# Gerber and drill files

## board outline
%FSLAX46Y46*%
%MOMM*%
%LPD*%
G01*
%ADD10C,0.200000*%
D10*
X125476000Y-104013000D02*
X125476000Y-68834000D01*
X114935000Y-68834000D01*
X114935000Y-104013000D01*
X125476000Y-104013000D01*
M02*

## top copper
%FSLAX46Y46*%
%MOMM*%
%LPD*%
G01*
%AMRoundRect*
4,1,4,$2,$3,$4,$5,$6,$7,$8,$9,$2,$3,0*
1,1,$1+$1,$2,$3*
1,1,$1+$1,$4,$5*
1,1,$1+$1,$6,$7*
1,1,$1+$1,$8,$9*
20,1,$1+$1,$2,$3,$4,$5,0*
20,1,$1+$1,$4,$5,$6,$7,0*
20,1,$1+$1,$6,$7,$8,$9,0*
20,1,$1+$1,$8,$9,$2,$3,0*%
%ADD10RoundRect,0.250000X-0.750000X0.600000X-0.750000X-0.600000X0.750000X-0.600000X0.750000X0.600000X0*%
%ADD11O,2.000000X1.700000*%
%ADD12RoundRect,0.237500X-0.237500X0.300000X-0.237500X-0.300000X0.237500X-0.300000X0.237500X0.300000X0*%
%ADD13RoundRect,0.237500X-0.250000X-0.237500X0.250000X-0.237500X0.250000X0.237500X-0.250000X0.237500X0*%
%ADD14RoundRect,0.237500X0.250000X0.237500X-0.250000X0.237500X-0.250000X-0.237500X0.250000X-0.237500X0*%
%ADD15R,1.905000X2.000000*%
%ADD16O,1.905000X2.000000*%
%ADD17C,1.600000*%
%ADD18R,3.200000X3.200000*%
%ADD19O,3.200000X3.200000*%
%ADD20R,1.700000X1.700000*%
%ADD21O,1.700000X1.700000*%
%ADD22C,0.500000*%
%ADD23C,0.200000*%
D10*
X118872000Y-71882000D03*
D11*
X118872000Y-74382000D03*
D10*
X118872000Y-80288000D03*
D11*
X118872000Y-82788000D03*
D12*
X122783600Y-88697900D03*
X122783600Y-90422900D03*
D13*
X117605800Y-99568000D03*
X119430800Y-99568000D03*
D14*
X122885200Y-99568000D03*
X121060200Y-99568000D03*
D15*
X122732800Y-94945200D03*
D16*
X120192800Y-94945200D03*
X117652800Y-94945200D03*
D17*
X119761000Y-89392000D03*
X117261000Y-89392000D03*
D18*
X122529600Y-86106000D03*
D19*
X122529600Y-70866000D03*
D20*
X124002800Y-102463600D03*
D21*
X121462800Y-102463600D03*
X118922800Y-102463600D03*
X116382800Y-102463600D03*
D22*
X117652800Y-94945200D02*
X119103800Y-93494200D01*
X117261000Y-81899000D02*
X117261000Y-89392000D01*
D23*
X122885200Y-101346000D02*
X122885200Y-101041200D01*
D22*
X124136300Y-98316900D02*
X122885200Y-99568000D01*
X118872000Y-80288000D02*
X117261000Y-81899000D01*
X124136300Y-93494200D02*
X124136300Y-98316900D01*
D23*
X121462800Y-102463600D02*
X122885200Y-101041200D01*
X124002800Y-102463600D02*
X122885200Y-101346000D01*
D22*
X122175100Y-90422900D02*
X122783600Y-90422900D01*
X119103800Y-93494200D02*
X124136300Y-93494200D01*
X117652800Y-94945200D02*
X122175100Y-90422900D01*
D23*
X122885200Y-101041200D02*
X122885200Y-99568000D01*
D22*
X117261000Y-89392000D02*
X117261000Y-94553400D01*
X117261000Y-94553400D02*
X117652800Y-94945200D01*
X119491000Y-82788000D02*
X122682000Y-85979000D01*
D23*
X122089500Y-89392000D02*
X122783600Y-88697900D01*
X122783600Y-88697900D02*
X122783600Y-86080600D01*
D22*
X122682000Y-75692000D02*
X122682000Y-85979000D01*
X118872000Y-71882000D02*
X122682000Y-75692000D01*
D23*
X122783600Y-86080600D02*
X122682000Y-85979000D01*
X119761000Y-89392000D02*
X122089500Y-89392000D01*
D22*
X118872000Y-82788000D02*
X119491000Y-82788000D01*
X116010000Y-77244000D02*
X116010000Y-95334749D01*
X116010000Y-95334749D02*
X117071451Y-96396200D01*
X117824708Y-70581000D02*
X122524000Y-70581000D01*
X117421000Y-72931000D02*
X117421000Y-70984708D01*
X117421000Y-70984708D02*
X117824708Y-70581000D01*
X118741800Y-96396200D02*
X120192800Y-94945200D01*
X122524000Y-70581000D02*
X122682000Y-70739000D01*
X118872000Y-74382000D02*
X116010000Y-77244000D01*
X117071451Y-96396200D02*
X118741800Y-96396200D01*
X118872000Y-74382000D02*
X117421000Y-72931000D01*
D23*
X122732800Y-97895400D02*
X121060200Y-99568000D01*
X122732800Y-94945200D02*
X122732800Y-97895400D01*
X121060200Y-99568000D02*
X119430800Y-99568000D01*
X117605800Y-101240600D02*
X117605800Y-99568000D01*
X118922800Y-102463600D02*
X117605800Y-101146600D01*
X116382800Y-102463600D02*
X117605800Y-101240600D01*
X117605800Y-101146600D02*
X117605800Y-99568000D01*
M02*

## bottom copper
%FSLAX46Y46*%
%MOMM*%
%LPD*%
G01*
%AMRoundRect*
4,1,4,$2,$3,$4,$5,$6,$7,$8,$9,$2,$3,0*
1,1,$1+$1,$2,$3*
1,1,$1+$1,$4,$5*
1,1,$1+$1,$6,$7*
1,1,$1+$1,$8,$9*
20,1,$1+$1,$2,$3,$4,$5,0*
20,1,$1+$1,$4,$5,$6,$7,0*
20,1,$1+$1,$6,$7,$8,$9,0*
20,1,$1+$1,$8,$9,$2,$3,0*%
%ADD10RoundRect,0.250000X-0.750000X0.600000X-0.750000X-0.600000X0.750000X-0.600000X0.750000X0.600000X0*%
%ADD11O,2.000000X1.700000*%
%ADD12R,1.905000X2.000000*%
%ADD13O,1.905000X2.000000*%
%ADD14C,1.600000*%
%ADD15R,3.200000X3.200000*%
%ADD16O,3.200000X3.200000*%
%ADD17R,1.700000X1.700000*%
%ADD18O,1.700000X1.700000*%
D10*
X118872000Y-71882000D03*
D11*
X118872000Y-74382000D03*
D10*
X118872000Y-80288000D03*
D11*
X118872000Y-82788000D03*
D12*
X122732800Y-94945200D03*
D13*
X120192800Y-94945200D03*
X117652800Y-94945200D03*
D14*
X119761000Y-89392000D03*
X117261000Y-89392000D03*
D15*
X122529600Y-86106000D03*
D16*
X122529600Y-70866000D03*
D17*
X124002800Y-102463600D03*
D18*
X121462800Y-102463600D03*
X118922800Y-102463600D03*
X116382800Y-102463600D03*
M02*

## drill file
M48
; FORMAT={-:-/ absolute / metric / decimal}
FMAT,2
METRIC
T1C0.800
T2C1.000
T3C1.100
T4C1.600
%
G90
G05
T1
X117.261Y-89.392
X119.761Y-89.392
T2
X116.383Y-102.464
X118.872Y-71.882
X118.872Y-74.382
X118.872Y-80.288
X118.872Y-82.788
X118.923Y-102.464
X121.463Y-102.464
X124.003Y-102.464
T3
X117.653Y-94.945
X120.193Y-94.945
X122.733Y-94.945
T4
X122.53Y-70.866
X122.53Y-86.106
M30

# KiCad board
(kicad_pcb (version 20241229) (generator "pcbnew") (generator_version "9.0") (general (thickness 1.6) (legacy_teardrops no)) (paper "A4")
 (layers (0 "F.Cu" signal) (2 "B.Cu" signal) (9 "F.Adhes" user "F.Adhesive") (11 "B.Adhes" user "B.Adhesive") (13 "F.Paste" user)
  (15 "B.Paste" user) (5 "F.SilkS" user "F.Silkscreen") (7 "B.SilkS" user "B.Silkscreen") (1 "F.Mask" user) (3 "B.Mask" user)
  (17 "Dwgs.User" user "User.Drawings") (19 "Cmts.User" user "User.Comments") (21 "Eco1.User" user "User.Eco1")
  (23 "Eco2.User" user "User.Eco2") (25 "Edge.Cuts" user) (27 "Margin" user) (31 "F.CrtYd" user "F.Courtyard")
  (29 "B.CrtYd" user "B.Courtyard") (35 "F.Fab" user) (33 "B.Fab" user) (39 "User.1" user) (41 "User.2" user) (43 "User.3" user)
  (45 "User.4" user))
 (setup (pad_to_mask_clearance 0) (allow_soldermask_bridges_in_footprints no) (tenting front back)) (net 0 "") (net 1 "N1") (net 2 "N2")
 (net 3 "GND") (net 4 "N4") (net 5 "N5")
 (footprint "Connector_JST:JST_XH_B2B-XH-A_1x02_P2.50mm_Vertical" (layer "F.Cu") (at 118.872 71.882 -90)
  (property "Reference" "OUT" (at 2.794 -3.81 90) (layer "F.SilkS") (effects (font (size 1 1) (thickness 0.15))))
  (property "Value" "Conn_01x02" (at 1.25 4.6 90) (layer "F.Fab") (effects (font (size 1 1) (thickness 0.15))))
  (pad "1" thru_hole roundrect (at 0 0 270) (size 1.7 2) (drill 1) (layers "*.Cu" "*.Mask") (remove_unused_layers no)
   (roundrect_rratio 0.147059) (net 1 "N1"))
  (pad "2" thru_hole oval (at 2.5 0 270) (size 1.7 2) (drill 1) (layers "*.Cu" "*.Mask") (remove_unused_layers no) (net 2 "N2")))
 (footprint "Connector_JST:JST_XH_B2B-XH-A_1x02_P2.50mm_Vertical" (layer "F.Cu") (at 118.872 80.288 -90)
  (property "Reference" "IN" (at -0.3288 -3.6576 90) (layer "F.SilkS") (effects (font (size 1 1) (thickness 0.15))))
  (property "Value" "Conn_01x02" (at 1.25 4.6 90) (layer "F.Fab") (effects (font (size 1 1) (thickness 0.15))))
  (pad "1" thru_hole roundrect (at 0 0 270) (size 1.7 2) (drill 1) (layers "*.Cu" "*.Mask") (remove_unused_layers no)
   (roundrect_rratio 0.147059) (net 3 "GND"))
  (pad "2" thru_hole oval (at 2.5 0 270) (size 1.7 2) (drill 1) (layers "*.Cu" "*.Mask") (remove_unused_layers no) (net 1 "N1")))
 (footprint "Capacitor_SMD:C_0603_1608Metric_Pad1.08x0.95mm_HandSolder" (layer "F.Cu") (at 122.7836 89.5604 -90)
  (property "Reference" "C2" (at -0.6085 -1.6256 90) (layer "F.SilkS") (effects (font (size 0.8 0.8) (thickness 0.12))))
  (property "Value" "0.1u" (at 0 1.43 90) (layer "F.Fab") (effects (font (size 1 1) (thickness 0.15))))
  (pad "1" smd roundrect (at -0.8625 0 270) (size 1.075 0.95) (layers "F.Cu" "F.Mask" "F.Paste") (roundrect_rratio 0.25) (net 1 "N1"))
  (pad "2" smd roundrect (at 0.8625 0 270) (size 1.075 0.95) (layers "F.Cu" "F.Mask" "F.Paste") (roundrect_rratio 0.25) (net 3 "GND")))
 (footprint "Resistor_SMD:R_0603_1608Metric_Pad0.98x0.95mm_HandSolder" (layer "F.Cu") (at 118.5183 99.568)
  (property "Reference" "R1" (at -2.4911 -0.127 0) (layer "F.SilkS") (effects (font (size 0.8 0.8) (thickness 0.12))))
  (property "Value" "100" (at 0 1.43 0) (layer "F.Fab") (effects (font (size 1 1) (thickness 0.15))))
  (pad "1" smd roundrect (at -0.9125 0) (size 0.975 0.95) (layers "F.Cu" "F.Mask" "F.Paste") (roundrect_rratio 0.25) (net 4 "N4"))
  (pad "2" smd roundrect (at 0.9125 0) (size 0.975 0.95) (layers "F.Cu" "F.Mask" "F.Paste") (roundrect_rratio 0.25) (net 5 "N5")))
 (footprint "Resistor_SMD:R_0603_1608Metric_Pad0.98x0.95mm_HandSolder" (layer "F.Cu") (at 121.9727 99.568 180)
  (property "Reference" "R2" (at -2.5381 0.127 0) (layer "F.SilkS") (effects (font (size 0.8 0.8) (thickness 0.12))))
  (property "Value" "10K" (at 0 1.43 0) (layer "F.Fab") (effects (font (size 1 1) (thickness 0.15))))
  (pad "1" smd roundrect (at -0.9125 0 180) (size 0.975 0.95) (layers "F.Cu" "F.Mask" "F.Paste") (roundrect_rratio 0.25) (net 3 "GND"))
  (pad "2" smd roundrect (at 0.9125 0 180) (size 0.975 0.95) (layers "F.Cu" "F.Mask" "F.Paste") (roundrect_rratio 0.25) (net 5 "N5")))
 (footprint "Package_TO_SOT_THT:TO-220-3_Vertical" (layer "F.Cu") (at 122.7328 94.9452 180)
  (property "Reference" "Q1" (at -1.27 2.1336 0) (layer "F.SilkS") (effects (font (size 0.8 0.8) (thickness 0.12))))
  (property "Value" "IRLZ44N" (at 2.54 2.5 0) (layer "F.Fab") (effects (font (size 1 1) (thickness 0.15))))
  (pad "1" thru_hole rect (at 0 0 180) (size 1.905 2) (drill 1.1) (layers "*.Cu" "*.Mask") (remove_unused_layers no) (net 5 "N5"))
  (pad "2" thru_hole oval (at 2.54 0 180) (size 1.905 2) (drill 1.1) (layers "*.Cu" "*.Mask") (remove_unused_layers no) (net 2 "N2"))
  (pad "3" thru_hole oval (at 5.08 0 180) (size 1.905 2) (drill 1.1) (layers "*.Cu" "*.Mask") (remove_unused_layers no) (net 3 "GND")))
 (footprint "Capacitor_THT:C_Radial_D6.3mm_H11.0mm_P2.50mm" (layer "F.Cu") (at 119.761 89.392 180)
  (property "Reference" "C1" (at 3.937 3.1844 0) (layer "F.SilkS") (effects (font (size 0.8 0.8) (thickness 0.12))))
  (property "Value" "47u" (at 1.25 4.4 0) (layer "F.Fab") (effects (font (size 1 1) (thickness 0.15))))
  (pad "1" thru_hole circle (at 0 0 180) (size 1.6 1.6) (drill 0.8) (layers "*.Cu" "*.Mask") (remove_unused_layers no) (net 1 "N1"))
  (pad "2" thru_hole circle (at 2.5 0 180) (size 1.6 1.6) (drill 0.8) (layers "*.Cu" "*.Mask") (remove_unused_layers no) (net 3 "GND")))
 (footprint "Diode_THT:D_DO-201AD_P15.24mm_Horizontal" (layer "B.Cu") (at 122.5296 86.106 90)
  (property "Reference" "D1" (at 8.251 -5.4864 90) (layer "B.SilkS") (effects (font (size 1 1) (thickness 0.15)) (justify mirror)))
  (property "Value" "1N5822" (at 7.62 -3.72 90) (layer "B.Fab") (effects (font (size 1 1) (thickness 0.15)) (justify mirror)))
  (pad "1" thru_hole rect (at 0 0 90) (size 3.2 3.2) (drill 1.6) (layers "*.Cu" "*.Mask") (remove_unused_layers no) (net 1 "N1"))
  (pad "2" thru_hole oval (at 15.24 0 90) (size 3.2 3.2) (drill 1.6) (layers "*.Cu" "*.Mask") (remove_unused_layers no) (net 2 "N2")))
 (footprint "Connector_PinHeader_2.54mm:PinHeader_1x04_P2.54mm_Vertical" (layer "B.Cu") (at 124.0028 102.4636 90)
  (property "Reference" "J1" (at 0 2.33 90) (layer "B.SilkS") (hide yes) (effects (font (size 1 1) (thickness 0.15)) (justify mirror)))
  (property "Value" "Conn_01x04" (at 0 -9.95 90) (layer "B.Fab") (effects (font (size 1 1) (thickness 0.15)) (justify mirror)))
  (pad "1" thru_hole rect (at 0 0 90) (size 1.7 1.7) (drill 1) (layers "*.Cu" "*.Mask") (remove_unused_layers no) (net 3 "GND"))
  (pad "2" thru_hole oval (at 0 -2.54 90) (size 1.7 1.7) (drill 1) (layers "*.Cu" "*.Mask") (remove_unused_layers no) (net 3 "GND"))
  (pad "3" thru_hole oval (at 0 -5.08 90) (size 1.7 1.7) (drill 1) (layers "*.Cu" "*.Mask") (remove_unused_layers no) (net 4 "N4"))
  (pad "4" thru_hole oval (at 0 -7.62 90) (size 1.7 1.7) (drill 1) (layers "*.Cu" "*.Mask") (remove_unused_layers no) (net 4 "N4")))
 (gr_poly
  (pts (xy 125.476 104.013) (xy 125.476 68.834) (xy 114.935 68.834) (xy 114.935 104.013)) (stroke (width 0.2) (type solid)) (fill no)
  (layer "Edge.Cuts"))
 (segment (start 117.6528 94.9452) (end 119.1038 93.4942) (width 0.5) (layer "F.Cu") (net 3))
 (segment (start 117.261 81.899) (end 117.261 89.392) (width 0.5) (layer "F.Cu") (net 3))
 (segment (start 122.8852 101.346) (end 122.8852 101.0412) (width 0.2) (layer "F.Cu") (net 3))
 (segment (start 124.1363 98.3169) (end 122.8852 99.568) (width 0.5) (layer "F.Cu") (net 3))
 (segment (start 118.872 80.288) (end 117.261 81.899) (width 0.5) (layer "F.Cu") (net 3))
 (segment (start 124.1363 93.4942) (end 124.1363 98.3169) (width 0.5) (layer "F.Cu") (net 3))
 (segment (start 121.4628 102.4636) (end 122.8852 101.0412) (width 0.2) (layer "F.Cu") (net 3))
 (segment (start 124.0028 102.4636) (end 122.8852 101.346) (width 0.2) (layer "F.Cu") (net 3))
 (segment (start 122.1751 90.4229) (end 122.7836 90.4229) (width 0.5) (layer "F.Cu") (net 3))
 (segment (start 119.1038 93.4942) (end 124.1363 93.4942) (width 0.5) (layer "F.Cu") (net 3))
 (segment (start 117.6528 94.9452) (end 122.1751 90.4229) (width 0.5) (layer "F.Cu") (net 3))
 (segment (start 122.8852 101.0412) (end 122.8852 99.568) (width 0.2) (layer "F.Cu") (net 3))
 (segment (start 117.261 89.392) (end 117.261 94.5534) (width 0.5) (layer "F.Cu") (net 3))
 (segment (start 117.261 94.5534) (end 117.6528 94.9452) (width 0.5) (layer "F.Cu") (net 3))
 (segment (start 119.491 82.788) (end 122.682 85.979) (width 0.5) (layer "F.Cu") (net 1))
 (segment (start 122.0895 89.392) (end 122.7836 88.6979) (width 0.2) (layer "F.Cu") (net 1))
 (segment (start 122.7836 88.6979) (end 122.7836 86.0806) (width 0.2) (layer "F.Cu") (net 1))
 (segment (start 122.682 75.692) (end 122.682 85.979) (width 0.5) (layer "F.Cu") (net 1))
 (segment (start 118.872 71.882) (end 122.682 75.692) (width 0.5) (layer "F.Cu") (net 1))
 (segment (start 122.7836 86.0806) (end 122.682 85.979) (width 0.2) (layer "F.Cu") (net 1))
 (segment (start 119.761 89.392) (end 122.0895 89.392) (width 0.2) (layer "F.Cu") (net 1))
 (segment (start 118.872 82.788) (end 119.491 82.788) (width 0.5) (layer "F.Cu") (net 1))
 (segment (start 116.01 77.244) (end 116.01 95.334749) (width 0.5) (layer "F.Cu") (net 2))
 (segment (start 116.01 95.334749) (end 117.071451 96.3962) (width 0.5) (layer "F.Cu") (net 2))
 (segment (start 117.824708 70.581) (end 122.524 70.581) (width 0.5) (layer "F.Cu") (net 2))
 (segment (start 117.421 72.931) (end 117.421 70.984708) (width 0.5) (layer "F.Cu") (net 2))
 (segment (start 117.421 70.984708) (end 117.824708 70.581) (width 0.5) (layer "F.Cu") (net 2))
 (segment (start 118.7418 96.3962) (end 120.1928 94.9452) (width 0.5) (layer "F.Cu") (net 2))
 (segment (start 122.524 70.581) (end 122.682 70.739) (width 0.5) (layer "F.Cu") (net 2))
 (segment (start 118.872 74.382) (end 116.01 77.244) (width 0.5) (layer "F.Cu") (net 2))
 (segment (start 117.071451 96.3962) (end 118.7418 96.3962) (width 0.5) (layer "F.Cu") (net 2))
 (segment (start 118.872 74.382) (end 117.421 72.931) (width 0.5) (layer "F.Cu") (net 2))
 (segment (start 122.7328 97.8954) (end 121.0602 99.568) (width 0.2) (layer "F.Cu") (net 5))
 (segment (start 122.7328 94.9452) (end 122.7328 97.8954) (width 0.2) (layer "F.Cu") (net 5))
 (segment (start 121.0602 99.568) (end 119.4308 99.568) (width 0.2) (layer "F.Cu") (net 5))
 (segment (start 117.6058 101.2406) (end 117.6058 99.568) (width 0.2) (layer "F.Cu") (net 4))
 (segment (start 118.9228 102.4636) (end 117.6058 101.1466) (width 0.2) (layer "F.Cu") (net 4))
 (segment (start 116.3828 102.4636) (end 117.6058 101.2406) (width 0.2) (layer "F.Cu") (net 4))
 (segment (start 117.6058 101.1466) (end 117.6058 99.568) (width 0.2) (layer "F.Cu") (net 4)))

